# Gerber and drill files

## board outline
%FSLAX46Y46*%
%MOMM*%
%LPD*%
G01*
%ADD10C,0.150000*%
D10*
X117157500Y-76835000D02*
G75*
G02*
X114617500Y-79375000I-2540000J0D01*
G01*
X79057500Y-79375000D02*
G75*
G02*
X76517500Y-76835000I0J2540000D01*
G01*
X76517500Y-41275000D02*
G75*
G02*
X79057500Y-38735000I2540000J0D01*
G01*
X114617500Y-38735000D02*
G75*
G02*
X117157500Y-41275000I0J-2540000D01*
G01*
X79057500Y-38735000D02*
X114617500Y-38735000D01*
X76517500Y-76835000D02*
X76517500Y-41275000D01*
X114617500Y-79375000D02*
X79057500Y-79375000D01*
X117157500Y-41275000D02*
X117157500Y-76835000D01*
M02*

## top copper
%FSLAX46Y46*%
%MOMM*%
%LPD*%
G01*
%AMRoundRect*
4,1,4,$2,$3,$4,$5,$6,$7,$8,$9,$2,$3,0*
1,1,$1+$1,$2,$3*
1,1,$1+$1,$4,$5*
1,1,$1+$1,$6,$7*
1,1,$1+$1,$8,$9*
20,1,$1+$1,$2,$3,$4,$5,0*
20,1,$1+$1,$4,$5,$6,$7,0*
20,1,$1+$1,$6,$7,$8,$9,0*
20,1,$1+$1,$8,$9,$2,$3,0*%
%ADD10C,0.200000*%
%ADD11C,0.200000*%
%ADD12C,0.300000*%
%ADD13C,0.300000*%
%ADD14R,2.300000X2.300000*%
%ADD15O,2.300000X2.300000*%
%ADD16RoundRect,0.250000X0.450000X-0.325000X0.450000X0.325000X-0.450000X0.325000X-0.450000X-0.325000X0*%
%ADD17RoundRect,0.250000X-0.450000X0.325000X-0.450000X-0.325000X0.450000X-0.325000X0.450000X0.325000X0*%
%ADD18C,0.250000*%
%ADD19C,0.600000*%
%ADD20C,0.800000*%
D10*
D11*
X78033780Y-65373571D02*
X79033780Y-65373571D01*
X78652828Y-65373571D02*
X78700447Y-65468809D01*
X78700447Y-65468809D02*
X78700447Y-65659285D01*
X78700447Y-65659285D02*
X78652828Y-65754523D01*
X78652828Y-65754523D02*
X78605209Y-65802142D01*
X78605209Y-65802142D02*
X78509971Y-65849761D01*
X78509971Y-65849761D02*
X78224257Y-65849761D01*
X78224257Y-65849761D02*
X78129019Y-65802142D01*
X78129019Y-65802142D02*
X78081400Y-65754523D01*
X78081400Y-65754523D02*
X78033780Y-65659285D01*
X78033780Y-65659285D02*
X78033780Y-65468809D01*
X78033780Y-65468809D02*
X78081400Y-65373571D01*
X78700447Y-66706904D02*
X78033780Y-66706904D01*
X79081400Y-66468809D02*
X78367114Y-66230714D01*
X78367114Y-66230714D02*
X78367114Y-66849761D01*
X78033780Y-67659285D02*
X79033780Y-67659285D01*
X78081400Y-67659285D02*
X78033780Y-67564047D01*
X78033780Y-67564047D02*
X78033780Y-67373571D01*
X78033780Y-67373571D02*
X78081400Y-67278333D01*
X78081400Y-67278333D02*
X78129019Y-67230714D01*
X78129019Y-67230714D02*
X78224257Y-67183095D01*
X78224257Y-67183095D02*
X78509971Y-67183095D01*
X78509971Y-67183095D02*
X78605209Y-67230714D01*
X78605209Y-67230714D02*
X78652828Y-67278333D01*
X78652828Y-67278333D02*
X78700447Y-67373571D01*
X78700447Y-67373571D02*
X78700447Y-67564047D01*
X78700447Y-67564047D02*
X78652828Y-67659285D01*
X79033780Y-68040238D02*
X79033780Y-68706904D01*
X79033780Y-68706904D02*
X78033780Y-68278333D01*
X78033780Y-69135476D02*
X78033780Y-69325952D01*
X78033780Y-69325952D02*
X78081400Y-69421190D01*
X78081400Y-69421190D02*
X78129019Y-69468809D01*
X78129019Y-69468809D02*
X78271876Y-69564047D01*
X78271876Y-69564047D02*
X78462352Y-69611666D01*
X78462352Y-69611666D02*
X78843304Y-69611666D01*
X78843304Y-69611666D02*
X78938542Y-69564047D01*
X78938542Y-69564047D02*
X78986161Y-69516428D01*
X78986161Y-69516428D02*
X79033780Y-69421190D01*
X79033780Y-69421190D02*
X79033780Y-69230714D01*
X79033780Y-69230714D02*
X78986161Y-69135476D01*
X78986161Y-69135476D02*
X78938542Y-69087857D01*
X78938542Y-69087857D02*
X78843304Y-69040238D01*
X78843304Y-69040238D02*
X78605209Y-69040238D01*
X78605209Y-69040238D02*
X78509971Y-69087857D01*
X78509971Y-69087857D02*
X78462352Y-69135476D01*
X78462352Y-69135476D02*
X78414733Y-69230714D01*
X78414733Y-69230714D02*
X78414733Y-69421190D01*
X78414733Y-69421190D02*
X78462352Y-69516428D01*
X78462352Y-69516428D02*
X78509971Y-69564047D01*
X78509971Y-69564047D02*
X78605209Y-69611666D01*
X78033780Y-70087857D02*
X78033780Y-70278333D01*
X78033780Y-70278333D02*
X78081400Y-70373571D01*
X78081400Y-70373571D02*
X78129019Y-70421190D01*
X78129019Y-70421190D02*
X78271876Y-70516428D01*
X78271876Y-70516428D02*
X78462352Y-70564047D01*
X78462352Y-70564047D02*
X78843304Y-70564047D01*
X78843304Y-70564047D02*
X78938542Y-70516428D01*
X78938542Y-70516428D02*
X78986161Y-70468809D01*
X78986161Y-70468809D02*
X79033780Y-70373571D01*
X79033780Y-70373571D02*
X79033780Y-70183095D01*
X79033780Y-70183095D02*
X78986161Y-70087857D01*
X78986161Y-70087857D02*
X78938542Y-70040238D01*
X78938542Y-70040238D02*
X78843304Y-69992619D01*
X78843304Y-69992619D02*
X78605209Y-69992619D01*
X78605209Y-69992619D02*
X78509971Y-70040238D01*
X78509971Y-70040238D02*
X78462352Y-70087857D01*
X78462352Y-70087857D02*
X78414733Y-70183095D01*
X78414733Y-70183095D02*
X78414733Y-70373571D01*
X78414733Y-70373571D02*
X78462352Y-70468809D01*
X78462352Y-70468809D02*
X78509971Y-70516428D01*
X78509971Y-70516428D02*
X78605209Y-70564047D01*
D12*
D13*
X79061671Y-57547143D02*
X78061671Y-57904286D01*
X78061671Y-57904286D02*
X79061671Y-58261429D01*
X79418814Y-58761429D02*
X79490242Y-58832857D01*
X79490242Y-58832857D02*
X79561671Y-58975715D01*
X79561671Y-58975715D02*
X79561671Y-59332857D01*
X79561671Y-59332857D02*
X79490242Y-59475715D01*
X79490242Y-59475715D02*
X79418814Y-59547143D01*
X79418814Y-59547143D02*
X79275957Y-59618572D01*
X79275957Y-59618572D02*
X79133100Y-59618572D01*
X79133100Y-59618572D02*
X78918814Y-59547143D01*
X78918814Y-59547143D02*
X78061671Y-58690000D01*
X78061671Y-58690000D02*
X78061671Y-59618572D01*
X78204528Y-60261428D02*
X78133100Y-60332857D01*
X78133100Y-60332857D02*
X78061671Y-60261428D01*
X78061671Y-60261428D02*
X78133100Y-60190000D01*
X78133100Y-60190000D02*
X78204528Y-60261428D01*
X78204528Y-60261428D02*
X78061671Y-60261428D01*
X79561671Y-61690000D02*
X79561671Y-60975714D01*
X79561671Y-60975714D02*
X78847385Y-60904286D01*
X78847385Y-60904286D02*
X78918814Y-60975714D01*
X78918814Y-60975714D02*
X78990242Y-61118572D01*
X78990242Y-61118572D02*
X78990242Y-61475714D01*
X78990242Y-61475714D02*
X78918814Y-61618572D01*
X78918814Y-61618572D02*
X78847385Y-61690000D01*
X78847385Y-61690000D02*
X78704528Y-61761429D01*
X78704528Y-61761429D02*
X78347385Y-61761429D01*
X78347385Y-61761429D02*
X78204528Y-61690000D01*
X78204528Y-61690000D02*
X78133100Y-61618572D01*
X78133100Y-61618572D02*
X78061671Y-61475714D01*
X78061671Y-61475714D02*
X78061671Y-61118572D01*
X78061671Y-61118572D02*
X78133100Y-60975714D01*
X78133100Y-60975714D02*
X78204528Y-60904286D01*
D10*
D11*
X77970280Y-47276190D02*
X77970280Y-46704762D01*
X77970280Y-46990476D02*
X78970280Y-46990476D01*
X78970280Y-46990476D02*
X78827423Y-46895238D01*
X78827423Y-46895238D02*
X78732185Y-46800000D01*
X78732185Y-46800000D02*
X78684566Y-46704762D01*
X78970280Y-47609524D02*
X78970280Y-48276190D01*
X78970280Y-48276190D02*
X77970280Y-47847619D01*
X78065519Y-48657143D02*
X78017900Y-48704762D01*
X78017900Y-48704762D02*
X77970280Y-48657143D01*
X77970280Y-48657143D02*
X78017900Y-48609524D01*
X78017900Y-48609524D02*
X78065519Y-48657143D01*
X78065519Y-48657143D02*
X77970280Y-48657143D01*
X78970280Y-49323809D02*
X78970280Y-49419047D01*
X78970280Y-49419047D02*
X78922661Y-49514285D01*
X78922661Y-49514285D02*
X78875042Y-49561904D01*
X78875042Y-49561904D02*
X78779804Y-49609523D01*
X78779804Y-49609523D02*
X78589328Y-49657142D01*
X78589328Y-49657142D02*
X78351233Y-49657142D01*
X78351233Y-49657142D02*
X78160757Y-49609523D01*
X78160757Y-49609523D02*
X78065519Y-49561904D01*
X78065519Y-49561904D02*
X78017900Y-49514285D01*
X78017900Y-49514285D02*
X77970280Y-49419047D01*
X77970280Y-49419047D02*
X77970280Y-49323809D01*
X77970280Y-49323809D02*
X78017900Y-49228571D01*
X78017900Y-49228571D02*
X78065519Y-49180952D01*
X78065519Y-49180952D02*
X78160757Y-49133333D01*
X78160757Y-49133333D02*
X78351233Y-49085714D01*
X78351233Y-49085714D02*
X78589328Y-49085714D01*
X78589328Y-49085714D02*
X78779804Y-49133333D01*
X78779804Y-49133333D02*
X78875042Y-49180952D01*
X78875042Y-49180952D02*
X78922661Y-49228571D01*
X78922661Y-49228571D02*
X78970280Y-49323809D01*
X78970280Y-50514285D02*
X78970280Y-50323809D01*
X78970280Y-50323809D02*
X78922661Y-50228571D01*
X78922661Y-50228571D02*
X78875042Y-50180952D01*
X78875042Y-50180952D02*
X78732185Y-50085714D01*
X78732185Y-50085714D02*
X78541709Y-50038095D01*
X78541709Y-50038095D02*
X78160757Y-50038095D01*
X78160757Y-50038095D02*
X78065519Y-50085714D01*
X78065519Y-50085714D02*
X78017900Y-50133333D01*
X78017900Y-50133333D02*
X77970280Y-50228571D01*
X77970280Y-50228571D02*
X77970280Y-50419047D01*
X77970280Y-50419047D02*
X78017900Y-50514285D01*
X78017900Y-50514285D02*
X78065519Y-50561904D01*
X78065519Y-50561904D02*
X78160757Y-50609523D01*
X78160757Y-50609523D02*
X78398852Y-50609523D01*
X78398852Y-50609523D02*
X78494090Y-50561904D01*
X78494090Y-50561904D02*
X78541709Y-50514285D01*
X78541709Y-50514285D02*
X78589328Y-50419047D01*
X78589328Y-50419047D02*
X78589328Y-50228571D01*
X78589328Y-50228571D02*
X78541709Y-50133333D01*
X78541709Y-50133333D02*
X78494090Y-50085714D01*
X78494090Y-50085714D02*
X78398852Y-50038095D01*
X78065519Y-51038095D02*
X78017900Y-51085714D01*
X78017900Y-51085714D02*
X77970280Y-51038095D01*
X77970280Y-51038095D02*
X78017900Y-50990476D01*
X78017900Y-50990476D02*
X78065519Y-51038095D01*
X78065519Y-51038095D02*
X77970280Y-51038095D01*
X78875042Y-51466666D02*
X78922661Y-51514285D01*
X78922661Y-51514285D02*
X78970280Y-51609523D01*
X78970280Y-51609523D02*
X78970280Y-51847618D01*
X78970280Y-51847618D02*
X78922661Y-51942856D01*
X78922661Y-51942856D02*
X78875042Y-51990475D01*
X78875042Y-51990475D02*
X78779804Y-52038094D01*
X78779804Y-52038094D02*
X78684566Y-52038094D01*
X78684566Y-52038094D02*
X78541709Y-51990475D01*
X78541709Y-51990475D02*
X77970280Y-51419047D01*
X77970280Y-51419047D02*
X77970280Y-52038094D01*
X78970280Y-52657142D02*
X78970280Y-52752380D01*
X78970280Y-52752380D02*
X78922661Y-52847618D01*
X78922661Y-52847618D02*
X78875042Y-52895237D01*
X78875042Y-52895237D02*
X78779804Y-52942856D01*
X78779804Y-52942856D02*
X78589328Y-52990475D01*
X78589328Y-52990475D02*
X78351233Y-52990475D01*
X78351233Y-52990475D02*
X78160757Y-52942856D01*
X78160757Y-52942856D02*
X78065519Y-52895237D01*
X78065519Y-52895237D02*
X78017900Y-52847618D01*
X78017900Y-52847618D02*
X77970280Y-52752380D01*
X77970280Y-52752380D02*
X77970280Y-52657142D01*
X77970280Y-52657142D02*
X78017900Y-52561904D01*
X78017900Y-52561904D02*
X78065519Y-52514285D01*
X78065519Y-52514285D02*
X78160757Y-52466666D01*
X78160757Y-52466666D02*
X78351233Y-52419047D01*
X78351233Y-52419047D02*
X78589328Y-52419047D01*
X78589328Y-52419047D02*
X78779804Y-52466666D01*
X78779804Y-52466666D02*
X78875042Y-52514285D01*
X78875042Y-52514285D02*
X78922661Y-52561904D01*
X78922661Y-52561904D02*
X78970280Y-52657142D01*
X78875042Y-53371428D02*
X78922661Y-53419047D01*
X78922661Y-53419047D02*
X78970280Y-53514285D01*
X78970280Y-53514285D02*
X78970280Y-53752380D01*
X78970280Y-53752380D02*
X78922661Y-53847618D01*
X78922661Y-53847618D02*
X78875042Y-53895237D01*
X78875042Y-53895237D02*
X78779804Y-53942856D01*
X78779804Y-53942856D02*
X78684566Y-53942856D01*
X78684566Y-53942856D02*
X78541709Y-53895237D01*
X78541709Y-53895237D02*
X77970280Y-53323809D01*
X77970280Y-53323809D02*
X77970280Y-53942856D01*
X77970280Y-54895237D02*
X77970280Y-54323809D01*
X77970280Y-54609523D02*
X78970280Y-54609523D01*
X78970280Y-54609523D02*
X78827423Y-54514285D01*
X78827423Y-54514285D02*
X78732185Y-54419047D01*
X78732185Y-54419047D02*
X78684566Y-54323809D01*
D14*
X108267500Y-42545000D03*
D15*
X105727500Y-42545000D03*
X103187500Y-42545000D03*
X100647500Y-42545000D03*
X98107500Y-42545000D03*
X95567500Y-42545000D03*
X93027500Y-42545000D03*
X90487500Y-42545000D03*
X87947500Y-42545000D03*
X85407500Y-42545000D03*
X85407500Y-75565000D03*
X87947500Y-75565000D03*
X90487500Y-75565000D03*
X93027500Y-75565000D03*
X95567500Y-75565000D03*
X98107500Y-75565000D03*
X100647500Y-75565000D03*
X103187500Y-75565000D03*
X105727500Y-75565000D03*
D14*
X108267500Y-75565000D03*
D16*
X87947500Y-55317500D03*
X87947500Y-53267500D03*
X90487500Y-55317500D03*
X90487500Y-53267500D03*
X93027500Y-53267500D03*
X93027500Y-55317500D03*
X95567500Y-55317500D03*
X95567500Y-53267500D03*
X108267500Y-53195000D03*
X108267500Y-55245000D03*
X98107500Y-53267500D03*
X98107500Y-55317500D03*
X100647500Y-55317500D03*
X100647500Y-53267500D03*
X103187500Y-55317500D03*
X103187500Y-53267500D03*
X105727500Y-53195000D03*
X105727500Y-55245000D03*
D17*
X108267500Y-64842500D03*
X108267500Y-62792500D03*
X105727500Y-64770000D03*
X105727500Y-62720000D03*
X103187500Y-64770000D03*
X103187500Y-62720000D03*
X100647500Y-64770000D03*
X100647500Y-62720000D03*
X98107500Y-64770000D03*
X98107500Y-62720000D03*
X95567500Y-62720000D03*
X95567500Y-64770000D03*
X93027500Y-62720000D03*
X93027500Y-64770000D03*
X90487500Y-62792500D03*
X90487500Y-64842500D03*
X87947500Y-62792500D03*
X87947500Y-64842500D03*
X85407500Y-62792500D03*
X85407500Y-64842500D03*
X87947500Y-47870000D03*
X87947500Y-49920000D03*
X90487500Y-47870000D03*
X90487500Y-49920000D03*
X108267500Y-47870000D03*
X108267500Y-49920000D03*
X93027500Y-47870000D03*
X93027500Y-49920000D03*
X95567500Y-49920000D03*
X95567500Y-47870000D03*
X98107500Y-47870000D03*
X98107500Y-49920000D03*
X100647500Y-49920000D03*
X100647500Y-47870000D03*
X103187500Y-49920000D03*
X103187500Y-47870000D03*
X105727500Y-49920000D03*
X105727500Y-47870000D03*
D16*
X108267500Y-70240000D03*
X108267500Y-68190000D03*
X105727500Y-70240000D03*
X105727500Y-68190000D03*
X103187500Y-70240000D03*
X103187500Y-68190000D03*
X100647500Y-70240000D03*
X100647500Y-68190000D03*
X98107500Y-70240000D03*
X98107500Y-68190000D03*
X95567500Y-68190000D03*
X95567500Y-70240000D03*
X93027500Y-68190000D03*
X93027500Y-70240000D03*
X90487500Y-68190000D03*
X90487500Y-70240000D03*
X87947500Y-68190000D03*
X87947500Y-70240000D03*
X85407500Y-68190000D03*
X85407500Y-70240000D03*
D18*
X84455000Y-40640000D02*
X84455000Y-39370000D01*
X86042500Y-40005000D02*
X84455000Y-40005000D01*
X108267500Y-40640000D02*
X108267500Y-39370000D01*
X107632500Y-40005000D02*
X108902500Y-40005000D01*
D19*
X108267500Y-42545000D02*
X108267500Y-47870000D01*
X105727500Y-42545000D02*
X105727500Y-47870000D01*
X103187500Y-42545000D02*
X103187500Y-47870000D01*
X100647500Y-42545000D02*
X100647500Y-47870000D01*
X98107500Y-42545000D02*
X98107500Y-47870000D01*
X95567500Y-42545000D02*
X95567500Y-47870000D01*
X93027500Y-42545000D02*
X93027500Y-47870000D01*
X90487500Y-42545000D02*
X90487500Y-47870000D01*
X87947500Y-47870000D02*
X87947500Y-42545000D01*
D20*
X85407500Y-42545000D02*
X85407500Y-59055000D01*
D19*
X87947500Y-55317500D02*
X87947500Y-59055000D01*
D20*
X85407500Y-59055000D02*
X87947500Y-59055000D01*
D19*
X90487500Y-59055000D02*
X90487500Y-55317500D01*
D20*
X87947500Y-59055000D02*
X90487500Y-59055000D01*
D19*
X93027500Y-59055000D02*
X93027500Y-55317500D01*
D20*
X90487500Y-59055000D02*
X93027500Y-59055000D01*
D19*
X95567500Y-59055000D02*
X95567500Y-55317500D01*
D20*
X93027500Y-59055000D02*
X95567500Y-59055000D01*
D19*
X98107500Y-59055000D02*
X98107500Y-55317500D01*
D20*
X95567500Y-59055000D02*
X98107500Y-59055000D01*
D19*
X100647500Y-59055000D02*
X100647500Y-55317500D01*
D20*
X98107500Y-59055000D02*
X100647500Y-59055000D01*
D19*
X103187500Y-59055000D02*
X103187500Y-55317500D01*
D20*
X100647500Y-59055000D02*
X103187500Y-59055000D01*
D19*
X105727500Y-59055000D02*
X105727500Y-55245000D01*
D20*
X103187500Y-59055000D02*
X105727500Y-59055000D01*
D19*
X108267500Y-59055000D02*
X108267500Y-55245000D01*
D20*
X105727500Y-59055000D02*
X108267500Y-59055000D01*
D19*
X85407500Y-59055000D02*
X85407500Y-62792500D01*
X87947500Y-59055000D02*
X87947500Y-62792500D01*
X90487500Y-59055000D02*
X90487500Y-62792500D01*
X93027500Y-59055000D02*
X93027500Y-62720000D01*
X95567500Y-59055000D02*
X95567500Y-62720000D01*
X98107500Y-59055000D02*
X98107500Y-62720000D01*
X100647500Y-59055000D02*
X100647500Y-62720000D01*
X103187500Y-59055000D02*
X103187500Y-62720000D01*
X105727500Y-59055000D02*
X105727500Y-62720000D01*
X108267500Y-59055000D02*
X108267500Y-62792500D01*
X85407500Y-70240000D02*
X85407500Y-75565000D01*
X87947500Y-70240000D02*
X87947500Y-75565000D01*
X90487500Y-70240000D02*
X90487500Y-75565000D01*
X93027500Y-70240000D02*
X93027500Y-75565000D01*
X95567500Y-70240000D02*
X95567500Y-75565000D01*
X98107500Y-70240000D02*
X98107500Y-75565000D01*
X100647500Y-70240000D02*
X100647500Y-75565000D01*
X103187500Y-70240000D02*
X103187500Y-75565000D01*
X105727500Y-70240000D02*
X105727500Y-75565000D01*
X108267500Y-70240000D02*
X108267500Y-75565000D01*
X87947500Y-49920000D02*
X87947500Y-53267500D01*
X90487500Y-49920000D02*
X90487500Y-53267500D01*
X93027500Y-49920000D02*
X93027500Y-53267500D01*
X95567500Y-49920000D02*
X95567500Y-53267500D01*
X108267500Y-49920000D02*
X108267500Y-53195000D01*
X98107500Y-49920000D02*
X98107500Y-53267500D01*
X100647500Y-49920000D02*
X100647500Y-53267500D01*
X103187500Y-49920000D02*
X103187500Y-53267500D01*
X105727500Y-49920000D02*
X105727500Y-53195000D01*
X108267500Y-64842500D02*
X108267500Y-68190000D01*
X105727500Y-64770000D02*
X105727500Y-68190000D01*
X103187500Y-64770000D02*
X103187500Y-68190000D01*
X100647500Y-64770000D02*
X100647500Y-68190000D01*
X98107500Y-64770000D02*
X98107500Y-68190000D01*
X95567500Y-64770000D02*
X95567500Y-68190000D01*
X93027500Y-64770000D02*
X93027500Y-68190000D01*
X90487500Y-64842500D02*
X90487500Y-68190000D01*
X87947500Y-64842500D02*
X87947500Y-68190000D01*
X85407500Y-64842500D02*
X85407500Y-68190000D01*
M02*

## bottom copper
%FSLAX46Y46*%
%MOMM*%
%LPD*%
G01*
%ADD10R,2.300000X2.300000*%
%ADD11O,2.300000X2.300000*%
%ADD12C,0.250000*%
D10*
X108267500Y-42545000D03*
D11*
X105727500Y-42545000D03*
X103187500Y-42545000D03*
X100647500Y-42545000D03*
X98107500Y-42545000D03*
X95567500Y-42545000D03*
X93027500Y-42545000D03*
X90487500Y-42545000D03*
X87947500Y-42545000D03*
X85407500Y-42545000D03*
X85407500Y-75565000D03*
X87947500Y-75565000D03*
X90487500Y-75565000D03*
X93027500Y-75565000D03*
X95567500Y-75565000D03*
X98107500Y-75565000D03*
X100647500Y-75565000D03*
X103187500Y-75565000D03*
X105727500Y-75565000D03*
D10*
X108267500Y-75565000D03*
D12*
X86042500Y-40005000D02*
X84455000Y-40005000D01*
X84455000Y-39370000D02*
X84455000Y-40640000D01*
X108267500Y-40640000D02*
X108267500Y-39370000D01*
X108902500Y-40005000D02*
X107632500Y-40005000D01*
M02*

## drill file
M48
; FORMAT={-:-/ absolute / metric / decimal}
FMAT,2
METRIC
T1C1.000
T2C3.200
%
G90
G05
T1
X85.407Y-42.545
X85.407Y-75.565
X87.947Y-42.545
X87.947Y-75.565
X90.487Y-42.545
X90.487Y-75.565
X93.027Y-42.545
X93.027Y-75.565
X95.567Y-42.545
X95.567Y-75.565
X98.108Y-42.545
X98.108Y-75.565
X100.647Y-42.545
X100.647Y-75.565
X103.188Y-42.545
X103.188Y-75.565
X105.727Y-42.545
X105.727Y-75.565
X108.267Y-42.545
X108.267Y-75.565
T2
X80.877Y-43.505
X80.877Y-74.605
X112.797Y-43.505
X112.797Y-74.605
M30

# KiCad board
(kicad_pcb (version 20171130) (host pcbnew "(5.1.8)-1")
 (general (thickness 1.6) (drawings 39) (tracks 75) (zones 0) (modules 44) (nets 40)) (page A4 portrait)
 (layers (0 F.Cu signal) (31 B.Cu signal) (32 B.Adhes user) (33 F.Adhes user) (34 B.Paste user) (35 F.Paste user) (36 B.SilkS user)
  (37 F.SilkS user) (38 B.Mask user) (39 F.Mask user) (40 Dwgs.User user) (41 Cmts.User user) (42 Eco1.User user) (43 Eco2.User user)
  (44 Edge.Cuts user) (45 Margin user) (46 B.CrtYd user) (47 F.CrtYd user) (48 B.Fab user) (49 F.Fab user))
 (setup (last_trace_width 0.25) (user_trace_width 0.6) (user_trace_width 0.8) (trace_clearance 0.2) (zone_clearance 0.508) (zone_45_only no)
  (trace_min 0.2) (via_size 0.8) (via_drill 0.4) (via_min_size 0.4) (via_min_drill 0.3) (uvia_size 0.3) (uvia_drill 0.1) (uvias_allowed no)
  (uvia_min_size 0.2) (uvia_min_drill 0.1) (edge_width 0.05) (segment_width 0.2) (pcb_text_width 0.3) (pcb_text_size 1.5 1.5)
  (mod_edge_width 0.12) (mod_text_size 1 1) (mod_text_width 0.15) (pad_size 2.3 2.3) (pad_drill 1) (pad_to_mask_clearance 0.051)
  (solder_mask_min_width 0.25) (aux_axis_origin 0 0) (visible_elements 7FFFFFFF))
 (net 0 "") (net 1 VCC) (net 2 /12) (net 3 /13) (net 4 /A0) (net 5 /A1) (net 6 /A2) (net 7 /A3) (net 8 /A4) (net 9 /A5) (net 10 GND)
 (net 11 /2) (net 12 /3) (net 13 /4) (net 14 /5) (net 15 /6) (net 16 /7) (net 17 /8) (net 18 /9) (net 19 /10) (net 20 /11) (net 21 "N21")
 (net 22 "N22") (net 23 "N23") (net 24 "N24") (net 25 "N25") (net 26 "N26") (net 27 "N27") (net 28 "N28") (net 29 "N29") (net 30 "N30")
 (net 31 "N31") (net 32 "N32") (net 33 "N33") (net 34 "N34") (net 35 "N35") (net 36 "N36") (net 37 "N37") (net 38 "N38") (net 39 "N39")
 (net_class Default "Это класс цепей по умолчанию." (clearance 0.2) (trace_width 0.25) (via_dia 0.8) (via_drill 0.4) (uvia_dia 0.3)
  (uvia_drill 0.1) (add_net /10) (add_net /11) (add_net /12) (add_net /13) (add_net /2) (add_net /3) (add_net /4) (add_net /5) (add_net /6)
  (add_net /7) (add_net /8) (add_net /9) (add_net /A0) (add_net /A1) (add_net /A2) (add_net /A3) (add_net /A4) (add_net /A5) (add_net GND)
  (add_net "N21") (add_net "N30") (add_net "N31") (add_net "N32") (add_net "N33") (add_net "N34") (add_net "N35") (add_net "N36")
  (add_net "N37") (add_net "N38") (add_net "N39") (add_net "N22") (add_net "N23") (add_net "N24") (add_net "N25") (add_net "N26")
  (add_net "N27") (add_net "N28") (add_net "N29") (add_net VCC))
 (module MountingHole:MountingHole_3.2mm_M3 (layer F.Cu) (at 112.7975 43.505 270)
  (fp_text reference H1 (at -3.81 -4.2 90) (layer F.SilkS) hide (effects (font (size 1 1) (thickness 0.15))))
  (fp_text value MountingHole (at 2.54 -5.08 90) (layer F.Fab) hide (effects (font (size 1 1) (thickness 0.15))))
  (pad 1 np_thru_hole circle (at 0 0 270) (size 3.2 3.2) (drill 3.2) (layers *.Cu *.Mask)))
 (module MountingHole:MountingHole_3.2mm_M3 (layer F.Cu) (at 80.8775 43.505 270)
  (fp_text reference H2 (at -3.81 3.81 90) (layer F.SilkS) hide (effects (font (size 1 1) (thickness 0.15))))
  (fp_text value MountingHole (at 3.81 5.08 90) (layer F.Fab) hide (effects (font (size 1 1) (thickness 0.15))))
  (pad 1 np_thru_hole circle (at 0 0 270) (size 3.2 3.2) (drill 3.2) (layers *.Cu *.Mask)))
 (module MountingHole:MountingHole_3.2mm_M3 (layer F.Cu) (at 112.7975 74.605 270)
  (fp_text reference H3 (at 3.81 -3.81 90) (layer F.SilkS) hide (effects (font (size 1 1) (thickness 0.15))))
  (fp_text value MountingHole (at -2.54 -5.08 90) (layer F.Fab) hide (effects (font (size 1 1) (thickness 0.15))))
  (pad 1 np_thru_hole circle (at 0 0 270) (size 3.2 3.2) (drill 3.2) (layers *.Cu *.Mask)))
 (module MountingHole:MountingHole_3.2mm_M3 (layer F.Cu) (at 80.8775 74.605 270)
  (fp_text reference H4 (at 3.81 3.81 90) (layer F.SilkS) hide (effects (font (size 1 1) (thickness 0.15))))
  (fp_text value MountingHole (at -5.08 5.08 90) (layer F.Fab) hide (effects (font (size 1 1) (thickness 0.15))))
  (pad 1 np_thru_hole circle (at 0 0 270) (size 3.2 3.2) (drill 3.2) (layers *.Cu *.Mask)))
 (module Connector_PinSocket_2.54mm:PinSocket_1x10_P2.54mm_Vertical (layer F.Cu) (at 108.2675 42.545 270)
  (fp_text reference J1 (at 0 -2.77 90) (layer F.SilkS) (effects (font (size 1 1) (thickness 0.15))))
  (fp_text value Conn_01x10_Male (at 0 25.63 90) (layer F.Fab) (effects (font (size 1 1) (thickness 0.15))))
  (pad 1 thru_hole rect (at 0 0 270) (size 2.3 2.3) (drill 1) (layers *.Cu *.Mask) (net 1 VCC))
  (pad 2 thru_hole oval (at 0 2.54 270) (size 2.3 2.3) (drill 1) (layers *.Cu *.Mask) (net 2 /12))
  (pad 3 thru_hole oval (at 0 5.08 270) (size 2.3 2.3) (drill 1) (layers *.Cu *.Mask) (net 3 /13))
  (pad 4 thru_hole oval (at 0 7.62 270) (size 2.3 2.3) (drill 1) (layers *.Cu *.Mask) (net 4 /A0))
  (pad 5 thru_hole oval (at 0 10.16 270) (size 2.3 2.3) (drill 1) (layers *.Cu *.Mask) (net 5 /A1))
  (pad 6 thru_hole oval (at 0 12.7 270) (size 2.3 2.3) (drill 1) (layers *.Cu *.Mask) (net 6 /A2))
  (pad 7 thru_hole oval (at 0 15.24 270) (size 2.3 2.3) (drill 1) (layers *.Cu *.Mask) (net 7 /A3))
  (pad 8 thru_hole oval (at 0 17.78 270) (size 2.3 2.3) (drill 1) (layers *.Cu *.Mask) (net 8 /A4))
  (pad 9 thru_hole oval (at 0 20.32 270) (size 2.3 2.3) (drill 1) (layers *.Cu *.Mask) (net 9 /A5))
  (pad 10 thru_hole oval (at 0 22.86 270) (size 2.3 2.3) (drill 1) (layers *.Cu *.Mask) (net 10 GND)))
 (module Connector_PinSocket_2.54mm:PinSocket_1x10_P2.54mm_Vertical (layer F.Cu) (at 108.2675 75.565 270)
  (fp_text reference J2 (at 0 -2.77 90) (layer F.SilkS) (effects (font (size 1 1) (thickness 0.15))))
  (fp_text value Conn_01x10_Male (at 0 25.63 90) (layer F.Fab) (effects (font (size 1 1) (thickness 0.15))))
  (pad 10 thru_hole oval (at 0 22.86 270) (size 2.3 2.3) (drill 1) (layers *.Cu *.Mask) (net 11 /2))
  (pad 9 thru_hole oval (at 0 20.32 270) (size 2.3 2.3) (drill 1) (layers *.Cu *.Mask) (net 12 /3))
  (pad 8 thru_hole oval (at 0 17.78 270) (size 2.3 2.3) (drill 1) (layers *.Cu *.Mask) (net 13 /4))
  (pad 7 thru_hole oval (at 0 15.24 270) (size 2.3 2.3) (drill 1) (layers *.Cu *.Mask) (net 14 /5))
  (pad 6 thru_hole oval (at 0 12.7 270) (size 2.3 2.3) (drill 1) (layers *.Cu *.Mask) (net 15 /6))
  (pad 5 thru_hole oval (at 0 10.16 270) (size 2.3 2.3) (drill 1) (layers *.Cu *.Mask) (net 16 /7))
  (pad 4 thru_hole oval (at 0 7.62 270) (size 2.3 2.3) (drill 1) (layers *.Cu *.Mask) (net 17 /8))
  (pad 3 thru_hole oval (at 0 5.08 270) (size 2.3 2.3) (drill 1) (layers *.Cu *.Mask) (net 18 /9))
  (pad 2 thru_hole oval (at 0 2.54 270) (size 2.3 2.3) (drill 1) (layers *.Cu *.Mask) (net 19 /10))
  (pad 1 thru_hole rect (at 0 0 270) (size 2.3 2.3) (drill 1) (layers *.Cu *.Mask) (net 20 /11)))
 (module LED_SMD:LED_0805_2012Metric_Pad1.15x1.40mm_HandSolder (layer F.Cu) (at 87.9475 54.2925 90)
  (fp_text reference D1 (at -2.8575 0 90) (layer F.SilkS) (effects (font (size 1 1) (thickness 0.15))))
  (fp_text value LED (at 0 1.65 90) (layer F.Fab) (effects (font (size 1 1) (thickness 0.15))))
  (pad 1 smd roundrect (at -1.025 0 90) (size 1.15 1.4) (layers F.Cu F.Paste F.Mask) (roundrect_rratio 0.217391) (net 10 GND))
  (pad 2 smd roundrect (at 1.025 0 90) (size 1.15 1.4) (layers F.Cu F.Paste F.Mask) (roundrect_rratio 0.217391) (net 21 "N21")))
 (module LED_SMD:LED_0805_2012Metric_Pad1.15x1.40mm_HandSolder (layer F.Cu) (at 90.4875 54.2925 90)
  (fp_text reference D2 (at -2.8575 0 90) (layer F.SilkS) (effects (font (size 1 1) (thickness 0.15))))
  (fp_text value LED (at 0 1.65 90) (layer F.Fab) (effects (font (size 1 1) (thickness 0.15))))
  (pad 1 smd roundrect (at -1.025 0 90) (size 1.15 1.4) (layers F.Cu F.Paste F.Mask) (roundrect_rratio 0.217391) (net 10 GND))
  (pad 2 smd roundrect (at 1.025 0 90) (size 1.15 1.4) (layers F.Cu F.Paste F.Mask) (roundrect_rratio 0.217391) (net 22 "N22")))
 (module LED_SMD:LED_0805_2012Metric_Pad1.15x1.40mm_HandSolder (layer F.Cu) (at 93.0275 54.2925 90)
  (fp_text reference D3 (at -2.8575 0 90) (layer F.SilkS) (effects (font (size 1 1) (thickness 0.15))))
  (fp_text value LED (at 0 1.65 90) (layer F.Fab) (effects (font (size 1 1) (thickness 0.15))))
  (pad 2 smd roundrect (at 1.025 0 90) (size 1.15 1.4) (layers F.Cu F.Paste F.Mask) (roundrect_rratio 0.217391) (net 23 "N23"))
  (pad 1 smd roundrect (at -1.025 0 90) (size 1.15 1.4) (layers F.Cu F.Paste F.Mask) (roundrect_rratio 0.217391) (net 10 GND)))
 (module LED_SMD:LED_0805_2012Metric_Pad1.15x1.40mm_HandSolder (layer F.Cu) (at 95.5675 54.2925 90)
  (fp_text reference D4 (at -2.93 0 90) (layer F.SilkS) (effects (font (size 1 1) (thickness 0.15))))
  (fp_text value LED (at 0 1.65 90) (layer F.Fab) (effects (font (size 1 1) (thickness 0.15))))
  (pad 1 smd roundrect (at -1.025 0 90) (size 1.15 1.4) (layers F.Cu F.Paste F.Mask) (roundrect_rratio 0.217391) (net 10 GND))
  (pad 2 smd roundrect (at 1.025 0 90) (size 1.15 1.4) (layers F.Cu F.Paste F.Mask) (roundrect_rratio 0.217391) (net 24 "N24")))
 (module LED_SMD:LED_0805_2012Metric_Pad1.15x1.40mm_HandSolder (layer F.Cu) (at 108.2675 54.22 90)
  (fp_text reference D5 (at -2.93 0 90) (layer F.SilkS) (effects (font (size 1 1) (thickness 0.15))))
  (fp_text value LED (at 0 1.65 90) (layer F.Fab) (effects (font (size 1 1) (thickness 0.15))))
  (pad 2 smd roundrect (at 1.025 0 90) (size 1.15 1.4) (layers F.Cu F.Paste F.Mask) (roundrect_rratio 0.217391) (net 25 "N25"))
  (pad 1 smd roundrect (at -1.025 0 90) (size 1.15 1.4) (layers F.Cu F.Paste F.Mask) (roundrect_rratio 0.217391) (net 10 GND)))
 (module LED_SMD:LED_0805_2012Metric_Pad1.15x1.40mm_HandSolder (layer F.Cu) (at 98.1075 54.2925 90)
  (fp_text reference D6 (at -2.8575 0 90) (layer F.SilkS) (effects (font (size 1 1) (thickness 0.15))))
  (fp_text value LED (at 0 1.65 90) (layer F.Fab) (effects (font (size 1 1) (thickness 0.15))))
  (pad 2 smd roundrect (at 1.025 0 90) (size 1.15 1.4) (layers F.Cu F.Paste F.Mask) (roundrect_rratio 0.217391) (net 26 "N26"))
  (pad 1 smd roundrect (at -1.025 0 90) (size 1.15 1.4) (layers F.Cu F.Paste F.Mask) (roundrect_rratio 0.217391) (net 10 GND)))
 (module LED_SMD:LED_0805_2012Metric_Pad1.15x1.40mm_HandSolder (layer F.Cu) (at 100.6475 54.2925 90)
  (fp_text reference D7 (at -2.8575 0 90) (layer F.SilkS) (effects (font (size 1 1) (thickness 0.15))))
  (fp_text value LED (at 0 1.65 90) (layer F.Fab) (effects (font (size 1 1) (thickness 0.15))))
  (pad 1 smd roundrect (at -1.025 0 90) (size 1.15 1.4) (layers F.Cu F.Paste F.Mask) (roundrect_rratio 0.217391) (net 10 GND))
  (pad 2 smd roundrect (at 1.025 0 90) (size 1.15 1.4) (layers F.Cu F.Paste F.Mask) (roundrect_rratio 0.217391) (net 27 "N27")))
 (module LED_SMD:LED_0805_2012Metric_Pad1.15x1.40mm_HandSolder (layer F.Cu) (at 103.1875 54.2925 90)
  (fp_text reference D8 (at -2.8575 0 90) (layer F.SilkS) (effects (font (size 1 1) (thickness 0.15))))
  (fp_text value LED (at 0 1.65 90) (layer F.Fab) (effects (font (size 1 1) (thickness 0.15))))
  (pad 1 smd roundrect (at -1.025 0 90) (size 1.15 1.4) (layers F.Cu F.Paste F.Mask) (roundrect_rratio 0.217391) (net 10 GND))
  (pad 2 smd roundrect (at 1.025 0 90) (size 1.15 1.4) (layers F.Cu F.Paste F.Mask) (roundrect_rratio 0.217391) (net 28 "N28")))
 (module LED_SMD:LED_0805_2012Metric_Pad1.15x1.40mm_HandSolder (layer F.Cu) (at 105.7275 54.22 90)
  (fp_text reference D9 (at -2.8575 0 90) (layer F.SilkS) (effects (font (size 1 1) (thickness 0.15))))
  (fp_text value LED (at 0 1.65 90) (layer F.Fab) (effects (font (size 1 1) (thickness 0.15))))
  (pad 2 smd roundrect (at 1.025 0 90) (size 1.15 1.4) (layers F.Cu F.Paste F.Mask) (roundrect_rratio 0.217391) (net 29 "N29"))
  (pad 1 smd roundrect (at -1.025 0 90) (size 1.15 1.4) (layers F.Cu F.Paste F.Mask) (roundrect_rratio 0.217391) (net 10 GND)))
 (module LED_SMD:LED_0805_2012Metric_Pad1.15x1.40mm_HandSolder (layer F.Cu) (at 108.2675 63.8175 270)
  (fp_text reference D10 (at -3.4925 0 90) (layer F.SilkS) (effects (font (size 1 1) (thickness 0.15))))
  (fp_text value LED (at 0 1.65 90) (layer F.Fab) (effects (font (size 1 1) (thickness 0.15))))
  (pad 2 smd roundrect (at 1.025 0 270) (size 1.15 1.4) (layers F.Cu F.Paste F.Mask) (roundrect_rratio 0.217391) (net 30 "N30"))
  (pad 1 smd roundrect (at -1.025 0 270) (size 1.15 1.4) (layers F.Cu F.Paste F.Mask) (roundrect_rratio 0.217391) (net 10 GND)))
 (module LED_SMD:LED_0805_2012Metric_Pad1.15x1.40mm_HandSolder (layer F.Cu) (at 105.7275 63.745 270)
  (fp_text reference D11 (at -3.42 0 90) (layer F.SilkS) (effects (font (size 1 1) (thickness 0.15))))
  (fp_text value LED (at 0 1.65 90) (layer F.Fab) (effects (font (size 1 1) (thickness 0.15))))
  (pad 2 smd roundrect (at 1.025 0 270) (size 1.15 1.4) (layers F.Cu F.Paste F.Mask) (roundrect_rratio 0.217391) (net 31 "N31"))
  (pad 1 smd roundrect (at -1.025 0 270) (size 1.15 1.4) (layers F.Cu F.Paste F.Mask) (roundrect_rratio 0.217391) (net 10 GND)))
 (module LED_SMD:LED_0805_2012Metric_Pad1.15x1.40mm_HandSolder (layer F.Cu) (at 103.1875 63.745 270)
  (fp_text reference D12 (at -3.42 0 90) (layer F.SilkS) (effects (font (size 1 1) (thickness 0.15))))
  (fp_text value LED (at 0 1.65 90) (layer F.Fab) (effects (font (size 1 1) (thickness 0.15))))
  (pad 2 smd roundrect (at 1.025 0 270) (size 1.15 1.4) (layers F.Cu F.Paste F.Mask) (roundrect_rratio 0.217391) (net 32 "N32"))
  (pad 1 smd roundrect (at -1.025 0 270) (size 1.15 1.4) (layers F.Cu F.Paste F.Mask) (roundrect_rratio 0.217391) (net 10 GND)))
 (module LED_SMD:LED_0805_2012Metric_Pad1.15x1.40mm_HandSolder (layer F.Cu) (at 100.6475 63.745 270)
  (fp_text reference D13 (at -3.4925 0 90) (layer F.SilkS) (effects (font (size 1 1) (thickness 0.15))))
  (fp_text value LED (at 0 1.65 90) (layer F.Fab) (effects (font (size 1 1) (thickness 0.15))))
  (pad 2 smd roundrect (at 1.025 0 270) (size 1.15 1.4) (layers F.Cu F.Paste F.Mask) (roundrect_rratio 0.217391) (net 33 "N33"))
  (pad 1 smd roundrect (at -1.025 0 270) (size 1.15 1.4) (layers F.Cu F.Paste F.Mask) (roundrect_rratio 0.217391) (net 10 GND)))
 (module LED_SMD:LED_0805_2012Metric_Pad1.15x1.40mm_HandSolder (layer F.Cu) (at 98.1075 63.745 270)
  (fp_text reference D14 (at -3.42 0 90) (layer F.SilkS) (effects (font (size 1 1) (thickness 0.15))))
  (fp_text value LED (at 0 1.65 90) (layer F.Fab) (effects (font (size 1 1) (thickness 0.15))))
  (pad 2 smd roundrect (at 1.025 0 270) (size 1.15 1.4) (layers F.Cu F.Paste F.Mask) (roundrect_rratio 0.217391) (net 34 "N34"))
  (pad 1 smd roundrect (at -1.025 0 270) (size 1.15 1.4) (layers F.Cu F.Paste F.Mask) (roundrect_rratio 0.217391) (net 10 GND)))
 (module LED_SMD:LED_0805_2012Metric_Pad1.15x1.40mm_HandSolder (layer F.Cu) (at 95.5675 63.745 270)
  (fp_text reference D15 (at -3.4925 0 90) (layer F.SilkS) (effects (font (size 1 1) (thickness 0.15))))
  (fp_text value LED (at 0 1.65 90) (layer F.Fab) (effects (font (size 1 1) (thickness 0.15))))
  (pad 1 smd roundrect (at -1.025 0 270) (size 1.15 1.4) (layers F.Cu F.Paste F.Mask) (roundrect_rratio 0.217391) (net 10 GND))
  (pad 2 smd roundrect (at 1.025 0 270) (size 1.15 1.4) (layers F.Cu F.Paste F.Mask) (roundrect_rratio 0.217391) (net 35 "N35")))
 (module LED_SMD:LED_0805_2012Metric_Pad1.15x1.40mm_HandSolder (layer F.Cu) (at 93.0275 63.745 270)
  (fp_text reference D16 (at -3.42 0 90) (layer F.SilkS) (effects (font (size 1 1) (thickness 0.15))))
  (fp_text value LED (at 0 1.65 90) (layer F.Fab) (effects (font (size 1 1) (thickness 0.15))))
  (pad 1 smd roundrect (at -1.025 0 270) (size 1.15 1.4) (layers F.Cu F.Paste F.Mask) (roundrect_rratio 0.217391) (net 10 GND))
  (pad 2 smd roundrect (at 1.025 0 270) (size 1.15 1.4) (layers F.Cu F.Paste F.Mask) (roundrect_rratio 0.217391) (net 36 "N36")))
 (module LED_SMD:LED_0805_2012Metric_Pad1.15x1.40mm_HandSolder (layer F.Cu) (at 90.4875 63.8175 270)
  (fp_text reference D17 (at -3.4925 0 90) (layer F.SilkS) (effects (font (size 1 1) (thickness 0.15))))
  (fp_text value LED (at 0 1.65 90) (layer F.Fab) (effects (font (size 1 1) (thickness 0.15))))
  (pad 1 smd roundrect (at -1.025 0 270) (size 1.15 1.4) (layers F.Cu F.Paste F.Mask) (roundrect_rratio 0.217391) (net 10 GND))
  (pad 2 smd roundrect (at 1.025 0 270) (size 1.15 1.4) (layers F.Cu F.Paste F.Mask) (roundrect_rratio 0.217391) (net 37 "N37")))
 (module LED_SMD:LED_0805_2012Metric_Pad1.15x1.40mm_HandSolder (layer F.Cu) (at 87.9475 63.8175 270)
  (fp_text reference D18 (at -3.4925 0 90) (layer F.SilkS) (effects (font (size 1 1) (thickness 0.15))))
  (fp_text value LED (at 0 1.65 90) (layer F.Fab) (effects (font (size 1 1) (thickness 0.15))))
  (pad 1 smd roundrect (at -1.025 0 270) (size 1.15 1.4) (layers F.Cu F.Paste F.Mask) (roundrect_rratio 0.217391) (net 10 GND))
  (pad 2 smd roundrect (at 1.025 0 270) (size 1.15 1.4) (layers F.Cu F.Paste F.Mask) (roundrect_rratio 0.217391) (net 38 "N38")))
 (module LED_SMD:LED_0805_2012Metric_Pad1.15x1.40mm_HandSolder (layer F.Cu) (at 85.4075 63.8175 270)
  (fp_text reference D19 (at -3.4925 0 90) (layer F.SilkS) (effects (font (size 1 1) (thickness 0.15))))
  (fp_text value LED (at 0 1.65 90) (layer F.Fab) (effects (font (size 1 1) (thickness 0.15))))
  (pad 1 smd roundrect (at -1.025 0 270) (size 1.15 1.4) (layers F.Cu F.Paste F.Mask) (roundrect_rratio 0.217391) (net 10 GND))
  (pad 2 smd roundrect (at 1.025 0 270) (size 1.15 1.4) (layers F.Cu F.Paste F.Mask) (roundrect_rratio 0.217391) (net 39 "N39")))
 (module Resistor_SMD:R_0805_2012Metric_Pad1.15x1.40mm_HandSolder (layer F.Cu) (at 87.9475 48.895 270)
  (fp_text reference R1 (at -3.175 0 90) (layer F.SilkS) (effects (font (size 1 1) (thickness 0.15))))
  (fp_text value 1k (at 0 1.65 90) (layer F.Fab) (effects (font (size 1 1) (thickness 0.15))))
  (pad 1 smd roundrect (at -1.025 0 270) (size 1.15 1.4) (layers F.Cu F.Paste F.Mask) (roundrect_rratio 0.217391) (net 9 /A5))
  (pad 2 smd roundrect (at 1.025 0 270) (size 1.15 1.4) (layers F.Cu F.Paste F.Mask) (roundrect_rratio 0.217391) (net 21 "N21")))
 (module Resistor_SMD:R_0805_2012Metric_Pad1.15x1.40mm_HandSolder (layer F.Cu) (at 90.4875 48.895 270)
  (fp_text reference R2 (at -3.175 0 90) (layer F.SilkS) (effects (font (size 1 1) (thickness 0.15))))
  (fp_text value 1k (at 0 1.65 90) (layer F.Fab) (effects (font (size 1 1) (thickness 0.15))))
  (pad 1 smd roundrect (at -1.025 0 270) (size 1.15 1.4) (layers F.Cu F.Paste F.Mask) (roundrect_rratio 0.217391) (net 8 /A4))
  (pad 2 smd roundrect (at 1.025 0 270) (size 1.15 1.4) (layers F.Cu F.Paste F.Mask) (roundrect_rratio 0.217391) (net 22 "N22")))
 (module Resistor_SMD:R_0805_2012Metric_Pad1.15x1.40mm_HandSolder (layer F.Cu) (at 108.2675 48.895 270)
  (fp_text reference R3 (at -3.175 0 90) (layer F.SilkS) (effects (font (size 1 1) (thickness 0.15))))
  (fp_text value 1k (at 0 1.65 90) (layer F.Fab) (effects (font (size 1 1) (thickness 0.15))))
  (pad 1 smd roundrect (at -1.025 0 270) (size 1.15 1.4) (layers F.Cu F.Paste F.Mask) (roundrect_rratio 0.217391) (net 1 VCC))
  (pad 2 smd roundrect (at 1.025 0 270) (size 1.15 1.4) (layers F.Cu F.Paste F.Mask) (roundrect_rratio 0.217391) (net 25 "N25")))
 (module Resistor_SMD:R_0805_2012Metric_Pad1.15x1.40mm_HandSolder (layer F.Cu) (at 93.0275 48.895 270)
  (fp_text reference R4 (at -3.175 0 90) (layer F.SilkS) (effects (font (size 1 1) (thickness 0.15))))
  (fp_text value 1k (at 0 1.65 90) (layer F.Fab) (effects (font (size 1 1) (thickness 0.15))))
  (pad 1 smd roundrect (at -1.025 0 270) (size 1.15 1.4) (layers F.Cu F.Paste F.Mask) (roundrect_rratio 0.217391) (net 7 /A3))
  (pad 2 smd roundrect (at 1.025 0 270) (size 1.15 1.4) (layers F.Cu F.Paste F.Mask) (roundrect_rratio 0.217391) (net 23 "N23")))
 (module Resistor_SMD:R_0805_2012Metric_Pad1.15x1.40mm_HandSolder (layer F.Cu) (at 95.5675 48.895 270)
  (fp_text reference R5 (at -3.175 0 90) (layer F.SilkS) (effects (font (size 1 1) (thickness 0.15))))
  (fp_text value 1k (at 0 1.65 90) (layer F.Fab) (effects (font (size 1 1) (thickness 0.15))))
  (pad 2 smd roundrect (at 1.025 0 270) (size 1.15 1.4) (layers F.Cu F.Paste F.Mask) (roundrect_rratio 0.217391) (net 24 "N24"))
  (pad 1 smd roundrect (at -1.025 0 270) (size 1.15 1.4) (layers F.Cu F.Paste F.Mask) (roundrect_rratio 0.217391) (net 6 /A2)))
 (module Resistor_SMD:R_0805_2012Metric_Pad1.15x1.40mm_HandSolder (layer F.Cu) (at 98.1075 48.895 270)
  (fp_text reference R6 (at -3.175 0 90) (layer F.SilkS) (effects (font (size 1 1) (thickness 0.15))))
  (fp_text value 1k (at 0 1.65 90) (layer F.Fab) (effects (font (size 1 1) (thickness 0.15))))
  (pad 1 smd roundrect (at -1.025 0 270) (size 1.15 1.4) (layers F.Cu F.Paste F.Mask) (roundrect_rratio 0.217391) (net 5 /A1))
  (pad 2 smd roundrect (at 1.025 0 270) (size 1.15 1.4) (layers F.Cu F.Paste F.Mask) (roundrect_rratio 0.217391) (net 26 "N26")))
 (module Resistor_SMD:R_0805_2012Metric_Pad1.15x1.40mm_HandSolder (layer F.Cu) (at 100.6475 48.895 270)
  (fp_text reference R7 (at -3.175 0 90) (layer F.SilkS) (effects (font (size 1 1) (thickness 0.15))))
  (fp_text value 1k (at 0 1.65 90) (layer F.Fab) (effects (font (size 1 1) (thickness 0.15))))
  (pad 2 smd roundrect (at 1.025 0 270) (size 1.15 1.4) (layers F.Cu F.Paste F.Mask) (roundrect_rratio 0.217391) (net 27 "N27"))
  (pad 1 smd roundrect (at -1.025 0 270) (size 1.15 1.4) (layers F.Cu F.Paste F.Mask) (roundrect_rratio 0.217391) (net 4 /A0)))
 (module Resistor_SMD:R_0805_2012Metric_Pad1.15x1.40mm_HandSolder (layer F.Cu) (at 103.1875 48.895 270)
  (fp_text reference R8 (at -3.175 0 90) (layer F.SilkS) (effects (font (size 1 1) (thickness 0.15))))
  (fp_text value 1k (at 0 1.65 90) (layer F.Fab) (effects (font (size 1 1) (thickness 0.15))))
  (pad 2 smd roundrect (at 1.025 0 270) (size 1.15 1.4) (layers F.Cu F.Paste F.Mask) (roundrect_rratio 0.217391) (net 28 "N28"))
  (pad 1 smd roundrect (at -1.025 0 270) (size 1.15 1.4) (layers F.Cu F.Paste F.Mask) (roundrect_rratio 0.217391) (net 3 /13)))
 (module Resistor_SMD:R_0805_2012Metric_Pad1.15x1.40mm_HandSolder (layer F.Cu) (at 105.7275 48.895 270)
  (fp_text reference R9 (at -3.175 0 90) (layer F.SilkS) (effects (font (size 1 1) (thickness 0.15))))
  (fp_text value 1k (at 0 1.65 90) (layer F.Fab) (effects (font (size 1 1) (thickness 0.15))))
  (pad 2 smd roundrect (at 1.025 0 270) (size 1.15 1.4) (layers F.Cu F.Paste F.Mask) (roundrect_rratio 0.217391) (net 29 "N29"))
  (pad 1 smd roundrect (at -1.025 0 270) (size 1.15 1.4) (layers F.Cu F.Paste F.Mask) (roundrect_rratio 0.217391) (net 2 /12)))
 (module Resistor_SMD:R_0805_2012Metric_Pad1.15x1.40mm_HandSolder (layer F.Cu) (at 108.2675 69.215 90)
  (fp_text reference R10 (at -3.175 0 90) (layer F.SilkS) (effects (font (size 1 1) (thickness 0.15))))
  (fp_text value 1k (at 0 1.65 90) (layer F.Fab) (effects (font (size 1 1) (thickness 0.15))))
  (pad 1 smd roundrect (at -1.025 0 90) (size 1.15 1.4) (layers F.Cu F.Paste F.Mask) (roundrect_rratio 0.217391) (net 20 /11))
  (pad 2 smd roundrect (at 1.025 0 90) (size 1.15 1.4) (layers F.Cu F.Paste F.Mask) (roundrect_rratio 0.217391) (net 30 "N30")))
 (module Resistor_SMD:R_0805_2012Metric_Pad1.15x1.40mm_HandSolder (layer F.Cu) (at 105.7275 69.215 90)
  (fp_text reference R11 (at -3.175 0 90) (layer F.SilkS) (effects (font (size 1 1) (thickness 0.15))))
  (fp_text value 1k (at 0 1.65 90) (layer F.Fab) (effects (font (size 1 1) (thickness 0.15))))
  (pad 1 smd roundrect (at -1.025 0 90) (size 1.15 1.4) (layers F.Cu F.Paste F.Mask) (roundrect_rratio 0.217391) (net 19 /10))
  (pad 2 smd roundrect (at 1.025 0 90) (size 1.15 1.4) (layers F.Cu F.Paste F.Mask) (roundrect_rratio 0.217391) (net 31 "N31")))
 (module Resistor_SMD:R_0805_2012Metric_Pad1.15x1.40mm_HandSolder (layer F.Cu) (at 103.1875 69.215 90)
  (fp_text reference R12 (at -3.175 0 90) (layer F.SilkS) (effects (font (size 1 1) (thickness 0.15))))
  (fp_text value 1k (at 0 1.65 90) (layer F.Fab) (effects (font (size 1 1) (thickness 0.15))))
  (pad 1 smd roundrect (at -1.025 0 90) (size 1.15 1.4) (layers F.Cu F.Paste F.Mask) (roundrect_rratio 0.217391) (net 18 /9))
  (pad 2 smd roundrect (at 1.025 0 90) (size 1.15 1.4) (layers F.Cu F.Paste F.Mask) (roundrect_rratio 0.217391) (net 32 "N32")))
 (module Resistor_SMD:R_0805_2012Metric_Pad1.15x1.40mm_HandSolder (layer F.Cu) (at 100.6475 69.215 90)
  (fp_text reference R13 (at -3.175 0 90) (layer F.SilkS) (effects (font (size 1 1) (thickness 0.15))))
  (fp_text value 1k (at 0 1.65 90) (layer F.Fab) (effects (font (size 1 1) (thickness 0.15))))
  (pad 1 smd roundrect (at -1.025 0 90) (size 1.15 1.4) (layers F.Cu F.Paste F.Mask) (roundrect_rratio 0.217391) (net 17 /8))
  (pad 2 smd roundrect (at 1.025 0 90) (size 1.15 1.4) (layers F.Cu F.Paste F.Mask) (roundrect_rratio 0.217391) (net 33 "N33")))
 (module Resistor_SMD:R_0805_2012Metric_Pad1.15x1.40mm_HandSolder (layer F.Cu) (at 98.1075 69.215 90)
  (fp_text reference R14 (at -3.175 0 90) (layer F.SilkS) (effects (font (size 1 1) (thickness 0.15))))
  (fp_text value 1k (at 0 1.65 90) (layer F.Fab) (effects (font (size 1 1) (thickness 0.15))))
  (pad 1 smd roundrect (at -1.025 0 90) (size 1.15 1.4) (layers F.Cu F.Paste F.Mask) (roundrect_rratio 0.217391) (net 16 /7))
  (pad 2 smd roundrect (at 1.025 0 90) (size 1.15 1.4) (layers F.Cu F.Paste F.Mask) (roundrect_rratio 0.217391) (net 34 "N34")))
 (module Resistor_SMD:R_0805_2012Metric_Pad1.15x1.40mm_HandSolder (layer F.Cu) (at 95.5675 69.215 90)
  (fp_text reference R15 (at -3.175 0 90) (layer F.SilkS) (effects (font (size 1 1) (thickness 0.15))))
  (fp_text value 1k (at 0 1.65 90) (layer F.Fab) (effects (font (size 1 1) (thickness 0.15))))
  (pad 2 smd roundrect (at 1.025 0 90) (size 1.15 1.4) (layers F.Cu F.Paste F.Mask) (roundrect_rratio 0.217391) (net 35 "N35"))
  (pad 1 smd roundrect (at -1.025 0 90) (size 1.15 1.4) (layers F.Cu F.Paste F.Mask) (roundrect_rratio 0.217391) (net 15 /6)))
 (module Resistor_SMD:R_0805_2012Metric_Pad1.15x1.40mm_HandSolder (layer F.Cu) (at 93.0275 69.215 90)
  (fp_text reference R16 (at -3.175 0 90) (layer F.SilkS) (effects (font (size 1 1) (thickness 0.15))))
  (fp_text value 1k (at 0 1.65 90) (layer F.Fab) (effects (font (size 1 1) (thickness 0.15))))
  (pad 2 smd roundrect (at 1.025 0 90) (size 1.15 1.4) (layers F.Cu F.Paste F.Mask) (roundrect_rratio 0.217391) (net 36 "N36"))
  (pad 1 smd roundrect (at -1.025 0 90) (size 1.15 1.4) (layers F.Cu F.Paste F.Mask) (roundrect_rratio 0.217391) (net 14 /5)))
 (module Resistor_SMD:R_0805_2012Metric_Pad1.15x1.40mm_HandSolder (layer F.Cu) (at 90.4875 69.215 90)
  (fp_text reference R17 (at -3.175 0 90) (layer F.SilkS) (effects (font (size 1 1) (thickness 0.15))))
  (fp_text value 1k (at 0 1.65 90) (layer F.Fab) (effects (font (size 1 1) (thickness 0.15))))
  (pad 2 smd roundrect (at 1.025 0 90) (size 1.15 1.4) (layers F.Cu F.Paste F.Mask) (roundrect_rratio 0.217391) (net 37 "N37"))
  (pad 1 smd roundrect (at -1.025 0 90) (size 1.15 1.4) (layers F.Cu F.Paste F.Mask) (roundrect_rratio 0.217391) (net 13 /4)))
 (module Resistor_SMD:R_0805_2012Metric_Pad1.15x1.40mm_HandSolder (layer F.Cu) (at 87.9475 69.215 90)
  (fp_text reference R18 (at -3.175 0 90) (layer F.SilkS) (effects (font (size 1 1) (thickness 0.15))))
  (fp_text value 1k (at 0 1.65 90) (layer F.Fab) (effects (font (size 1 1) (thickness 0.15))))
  (pad 2 smd roundrect (at 1.025 0 90) (size 1.15 1.4) (layers F.Cu F.Paste F.Mask) (roundrect_rratio 0.217391) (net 38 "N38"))
  (pad 1 smd roundrect (at -1.025 0 90) (size 1.15 1.4) (layers F.Cu F.Paste F.Mask) (roundrect_rratio 0.217391) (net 12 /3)))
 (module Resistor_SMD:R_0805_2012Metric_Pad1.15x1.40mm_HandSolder (layer F.Cu) (at 85.4075 69.215 90)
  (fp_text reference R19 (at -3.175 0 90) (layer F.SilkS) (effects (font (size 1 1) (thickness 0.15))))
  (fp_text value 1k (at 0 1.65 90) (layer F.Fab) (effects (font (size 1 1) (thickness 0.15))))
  (pad 2 smd roundrect (at 1.025 0 90) (size 1.15 1.4) (layers F.Cu F.Paste F.Mask) (roundrect_rratio 0.217391) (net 39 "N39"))
  (pad 1 smd roundrect (at -1.025 0 90) (size 1.15 1.4) (layers F.Cu F.Paste F.Mask) (roundrect_rratio 0.217391) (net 11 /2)))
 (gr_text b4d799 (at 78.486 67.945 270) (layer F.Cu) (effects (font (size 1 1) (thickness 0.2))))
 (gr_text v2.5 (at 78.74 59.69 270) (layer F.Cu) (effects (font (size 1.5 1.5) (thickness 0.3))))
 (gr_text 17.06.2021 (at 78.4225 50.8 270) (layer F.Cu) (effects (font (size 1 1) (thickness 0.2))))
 (gr_arc (start 114.6175 76.835) (end 114.6175 79.375) (angle -90) (layer Edge.Cuts) (width 0.15))
 (gr_arc (start 79.0575 76.835) (end 76.5175 76.835) (angle -90) (layer Edge.Cuts) (width 0.15))
 (gr_arc (start 79.0575 41.275) (end 79.0575 38.735) (angle -90) (layer Edge.Cuts) (width 0.15))
 (gr_arc (start 114.6175 41.275) (end 117.1575 41.275) (angle -90) (layer Edge.Cuts) (width 0.15))
 (gr_line (start 79.0575 38.735) (end 114.6175 38.735) (layer Edge.Cuts) (width 0.15))
 (gr_line (start 76.5175 76.835) (end 76.5175 41.275) (layer Edge.Cuts) (width 0.15))
 (gr_line (start 114.6175 79.375) (end 79.0575 79.375) (layer Edge.Cuts) (width 0.15))
 (gr_line (start 117.1575 41.275) (end 117.1575 76.835) (layer Edge.Cuts) (width 0.15))
 (segment (start 86.0425 40.005) (end 84.455 40.005) (width 0.25) (layer B.Cu) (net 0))
 (segment (start 84.455 39.37) (end 84.455 40.64) (width 0.25) (layer B.Cu) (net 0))
 (segment (start 108.2675 40.64) (end 108.2675 39.37) (width 0.25) (layer B.Cu) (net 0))
 (segment (start 108.9025 40.005) (end 107.6325 40.005) (width 0.25) (layer B.Cu) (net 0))
 (segment (start 84.455 40.64) (end 84.455 39.37) (width 0.25) (layer F.Cu) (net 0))
 (segment (start 86.0425 40.005) (end 84.455 40.005) (width 0.25) (layer F.Cu) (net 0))
 (segment (start 108.2675 40.64) (end 108.2675 39.37) (width 0.25) (layer F.Cu) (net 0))
 (segment (start 107.6325 40.005) (end 108.9025 40.005) (width 0.25) (layer F.Cu) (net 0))
 (segment (start 108.2675 42.545) (end 108.2675 47.87) (width 0.6) (layer F.Cu) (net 1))
 (segment (start 105.7275 42.545) (end 105.7275 47.87) (width 0.6) (layer F.Cu) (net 2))
 (segment (start 103.1875 42.545) (end 103.1875 47.87) (width 0.6) (layer F.Cu) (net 3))
 (segment (start 100.6475 42.545) (end 100.6475 47.87) (width 0.6) (layer F.Cu) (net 4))
 (segment (start 98.1075 42.545) (end 98.1075 47.87) (width 0.6) (layer F.Cu) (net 5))
 (segment (start 95.5675 42.545) (end 95.5675 47.87) (width 0.6) (layer F.Cu) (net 6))
 (segment (start 93.0275 42.545) (end 93.0275 47.87) (width 0.6) (layer F.Cu) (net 7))
 (segment (start 90.4875 42.545) (end 90.4875 47.87) (width 0.6) (layer F.Cu) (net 8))
 (segment (start 87.9475 47.87) (end 87.9475 42.545) (width 0.6) (layer F.Cu) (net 9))
 (segment (start 85.4075 42.545) (end 85.4075 59.055) (width 0.8) (layer F.Cu) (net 10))
 (segment (start 87.9475 55.3175) (end 87.9475 59.055) (width 0.6) (layer F.Cu) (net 10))
 (segment (start 85.4075 59.055) (end 87.9475 59.055) (width 0.8) (layer F.Cu) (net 10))
 (segment (start 90.4875 59.055) (end 90.4875 55.3175) (width 0.6) (layer F.Cu) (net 10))
 (segment (start 87.9475 59.055) (end 90.4875 59.055) (width 0.8) (layer F.Cu) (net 10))
 (segment (start 93.0275 59.055) (end 93.0275 55.3175) (width 0.6) (layer F.Cu) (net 10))
 (segment (start 90.4875 59.055) (end 93.0275 59.055) (width 0.8) (layer F.Cu) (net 10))
 (segment (start 95.5675 59.055) (end 95.5675 55.3175) (width 0.6) (layer F.Cu) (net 10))
 (segment (start 93.0275 59.055) (end 95.5675 59.055) (width 0.8) (layer F.Cu) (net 10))
 (segment (start 98.1075 59.055) (end 98.1075 55.3175) (width 0.6) (layer F.Cu) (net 10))
 (segment (start 95.5675 59.055) (end 98.1075 59.055) (width 0.8) (layer F.Cu) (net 10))
 (segment (start 100.6475 59.055) (end 100.6475 55.3175) (width 0.6) (layer F.Cu) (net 10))
 (segment (start 98.1075 59.055) (end 100.6475 59.055) (width 0.8) (layer F.Cu) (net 10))
 (segment (start 103.1875 59.055) (end 103.1875 55.3175) (width 0.6) (layer F.Cu) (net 10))
 (segment (start 100.6475 59.055) (end 103.1875 59.055) (width 0.8) (layer F.Cu) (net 10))
 (segment (start 105.7275 59.055) (end 105.7275 55.245) (width 0.6) (layer F.Cu) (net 10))
 (segment (start 103.1875 59.055) (end 105.7275 59.055) (width 0.8) (layer F.Cu) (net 10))
 (segment (start 108.2675 59.055) (end 108.2675 55.245) (width 0.6) (layer F.Cu) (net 10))
 (segment (start 105.7275 59.055) (end 108.2675 59.055) (width 0.8) (layer F.Cu) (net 10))
 (segment (start 85.4075 59.055) (end 85.4075 62.7925) (width 0.6) (layer F.Cu) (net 10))
 (segment (start 87.9475 59.055) (end 87.9475 62.7925) (width 0.6) (layer F.Cu) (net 10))
 (segment (start 90.4875 59.055) (end 90.4875 62.7925) (width 0.6) (layer F.Cu) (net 10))
 (segment (start 93.0275 59.055) (end 93.0275 62.72) (width 0.6) (layer F.Cu) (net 10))
 (segment (start 95.5675 59.055) (end 95.5675 62.72) (width 0.6) (layer F.Cu) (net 10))
 (segment (start 98.1075 59.055) (end 98.1075 62.72) (width 0.6) (layer F.Cu) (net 10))
 (segment (start 100.6475 59.055) (end 100.6475 62.72) (width 0.6) (layer F.Cu) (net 10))
 (segment (start 103.1875 59.055) (end 103.1875 62.72) (width 0.6) (layer F.Cu) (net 10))
 (segment (start 105.7275 59.055) (end 105.7275 62.72) (width 0.6) (layer F.Cu) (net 10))
 (segment (start 108.2675 59.055) (end 108.2675 62.7925) (width 0.6) (layer F.Cu) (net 10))
 (segment (start 85.4075 70.24) (end 85.4075 75.565) (width 0.6) (layer F.Cu) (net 11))
 (segment (start 87.9475 70.24) (end 87.9475 75.565) (width 0.6) (layer F.Cu) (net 12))
 (segment (start 90.4875 70.24) (end 90.4875 75.565) (width 0.6) (layer F.Cu) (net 13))
 (segment (start 93.0275 70.24) (end 93.0275 75.565) (width 0.6) (layer F.Cu) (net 14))
 (segment (start 95.5675 70.24) (end 95.5675 75.565) (width 0.6) (layer F.Cu) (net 15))
 (segment (start 98.1075 70.24) (end 98.1075 75.565) (width 0.6) (layer F.Cu) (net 16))
 (segment (start 100.6475 70.24) (end 100.6475 75.565) (width 0.6) (layer F.Cu) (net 17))
 (segment (start 103.1875 70.24) (end 103.1875 75.565) (width 0.6) (layer F.Cu) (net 18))
 (segment (start 105.7275 70.24) (end 105.7275 75.565) (width 0.6) (layer F.Cu) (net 19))
 (segment (start 108.2675 70.24) (end 108.2675 75.565) (width 0.6) (layer F.Cu) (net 20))
 (segment (start 87.9475 49.92) (end 87.9475 53.2675) (width 0.6) (layer F.Cu) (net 21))
 (segment (start 90.4875 49.92) (end 90.4875 53.2675) (width 0.6) (layer F.Cu) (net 22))
 (segment (start 93.0275 49.92) (end 93.0275 53.2675) (width 0.6) (layer F.Cu) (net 23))
 (segment (start 95.5675 49.92) (end 95.5675 53.2675) (width 0.6) (layer F.Cu) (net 24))
 (segment (start 108.2675 49.92) (end 108.2675 53.195) (width 0.6) (layer F.Cu) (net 25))
 (segment (start 98.1075 49.92) (end 98.1075 53.2675) (width 0.6) (layer F.Cu) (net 26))
 (segment (start 100.6475 49.92) (end 100.6475 53.2675) (width 0.6) (layer F.Cu) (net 27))
 (segment (start 103.1875 49.92) (end 103.1875 53.2675) (width 0.6) (layer F.Cu) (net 28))
 (segment (start 105.7275 49.92) (end 105.7275 53.195) (width 0.6) (layer F.Cu) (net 29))
 (segment (start 108.2675 64.8425) (end 108.2675 68.19) (width 0.6) (layer F.Cu) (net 30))
 (segment (start 105.7275 64.77) (end 105.7275 68.19) (width 0.6) (layer F.Cu) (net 31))
 (segment (start 103.1875 64.77) (end 103.1875 68.19) (width 0.6) (layer F.Cu) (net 32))
 (segment (start 100.6475 64.77) (end 100.6475 68.19) (width 0.6) (layer F.Cu) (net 33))
 (segment (start 98.1075 64.77) (end 98.1075 68.19) (width 0.6) (layer F.Cu) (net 34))
 (segment (start 95.5675 64.77) (end 95.5675 68.19) (width 0.6) (layer F.Cu) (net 35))
 (segment (start 93.0275 64.77) (end 93.0275 68.19) (width 0.6) (layer F.Cu) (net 36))
 (segment (start 90.4875 64.8425) (end 90.4875 68.19) (width 0.6) (layer F.Cu) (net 37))
 (segment (start 87.9475 64.8425) (end 87.9475 68.19) (width 0.6) (layer F.Cu) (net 38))
 (segment (start 85.4075 64.8425) (end 85.4075 68.19) (width 0.6) (layer F.Cu) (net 39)))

